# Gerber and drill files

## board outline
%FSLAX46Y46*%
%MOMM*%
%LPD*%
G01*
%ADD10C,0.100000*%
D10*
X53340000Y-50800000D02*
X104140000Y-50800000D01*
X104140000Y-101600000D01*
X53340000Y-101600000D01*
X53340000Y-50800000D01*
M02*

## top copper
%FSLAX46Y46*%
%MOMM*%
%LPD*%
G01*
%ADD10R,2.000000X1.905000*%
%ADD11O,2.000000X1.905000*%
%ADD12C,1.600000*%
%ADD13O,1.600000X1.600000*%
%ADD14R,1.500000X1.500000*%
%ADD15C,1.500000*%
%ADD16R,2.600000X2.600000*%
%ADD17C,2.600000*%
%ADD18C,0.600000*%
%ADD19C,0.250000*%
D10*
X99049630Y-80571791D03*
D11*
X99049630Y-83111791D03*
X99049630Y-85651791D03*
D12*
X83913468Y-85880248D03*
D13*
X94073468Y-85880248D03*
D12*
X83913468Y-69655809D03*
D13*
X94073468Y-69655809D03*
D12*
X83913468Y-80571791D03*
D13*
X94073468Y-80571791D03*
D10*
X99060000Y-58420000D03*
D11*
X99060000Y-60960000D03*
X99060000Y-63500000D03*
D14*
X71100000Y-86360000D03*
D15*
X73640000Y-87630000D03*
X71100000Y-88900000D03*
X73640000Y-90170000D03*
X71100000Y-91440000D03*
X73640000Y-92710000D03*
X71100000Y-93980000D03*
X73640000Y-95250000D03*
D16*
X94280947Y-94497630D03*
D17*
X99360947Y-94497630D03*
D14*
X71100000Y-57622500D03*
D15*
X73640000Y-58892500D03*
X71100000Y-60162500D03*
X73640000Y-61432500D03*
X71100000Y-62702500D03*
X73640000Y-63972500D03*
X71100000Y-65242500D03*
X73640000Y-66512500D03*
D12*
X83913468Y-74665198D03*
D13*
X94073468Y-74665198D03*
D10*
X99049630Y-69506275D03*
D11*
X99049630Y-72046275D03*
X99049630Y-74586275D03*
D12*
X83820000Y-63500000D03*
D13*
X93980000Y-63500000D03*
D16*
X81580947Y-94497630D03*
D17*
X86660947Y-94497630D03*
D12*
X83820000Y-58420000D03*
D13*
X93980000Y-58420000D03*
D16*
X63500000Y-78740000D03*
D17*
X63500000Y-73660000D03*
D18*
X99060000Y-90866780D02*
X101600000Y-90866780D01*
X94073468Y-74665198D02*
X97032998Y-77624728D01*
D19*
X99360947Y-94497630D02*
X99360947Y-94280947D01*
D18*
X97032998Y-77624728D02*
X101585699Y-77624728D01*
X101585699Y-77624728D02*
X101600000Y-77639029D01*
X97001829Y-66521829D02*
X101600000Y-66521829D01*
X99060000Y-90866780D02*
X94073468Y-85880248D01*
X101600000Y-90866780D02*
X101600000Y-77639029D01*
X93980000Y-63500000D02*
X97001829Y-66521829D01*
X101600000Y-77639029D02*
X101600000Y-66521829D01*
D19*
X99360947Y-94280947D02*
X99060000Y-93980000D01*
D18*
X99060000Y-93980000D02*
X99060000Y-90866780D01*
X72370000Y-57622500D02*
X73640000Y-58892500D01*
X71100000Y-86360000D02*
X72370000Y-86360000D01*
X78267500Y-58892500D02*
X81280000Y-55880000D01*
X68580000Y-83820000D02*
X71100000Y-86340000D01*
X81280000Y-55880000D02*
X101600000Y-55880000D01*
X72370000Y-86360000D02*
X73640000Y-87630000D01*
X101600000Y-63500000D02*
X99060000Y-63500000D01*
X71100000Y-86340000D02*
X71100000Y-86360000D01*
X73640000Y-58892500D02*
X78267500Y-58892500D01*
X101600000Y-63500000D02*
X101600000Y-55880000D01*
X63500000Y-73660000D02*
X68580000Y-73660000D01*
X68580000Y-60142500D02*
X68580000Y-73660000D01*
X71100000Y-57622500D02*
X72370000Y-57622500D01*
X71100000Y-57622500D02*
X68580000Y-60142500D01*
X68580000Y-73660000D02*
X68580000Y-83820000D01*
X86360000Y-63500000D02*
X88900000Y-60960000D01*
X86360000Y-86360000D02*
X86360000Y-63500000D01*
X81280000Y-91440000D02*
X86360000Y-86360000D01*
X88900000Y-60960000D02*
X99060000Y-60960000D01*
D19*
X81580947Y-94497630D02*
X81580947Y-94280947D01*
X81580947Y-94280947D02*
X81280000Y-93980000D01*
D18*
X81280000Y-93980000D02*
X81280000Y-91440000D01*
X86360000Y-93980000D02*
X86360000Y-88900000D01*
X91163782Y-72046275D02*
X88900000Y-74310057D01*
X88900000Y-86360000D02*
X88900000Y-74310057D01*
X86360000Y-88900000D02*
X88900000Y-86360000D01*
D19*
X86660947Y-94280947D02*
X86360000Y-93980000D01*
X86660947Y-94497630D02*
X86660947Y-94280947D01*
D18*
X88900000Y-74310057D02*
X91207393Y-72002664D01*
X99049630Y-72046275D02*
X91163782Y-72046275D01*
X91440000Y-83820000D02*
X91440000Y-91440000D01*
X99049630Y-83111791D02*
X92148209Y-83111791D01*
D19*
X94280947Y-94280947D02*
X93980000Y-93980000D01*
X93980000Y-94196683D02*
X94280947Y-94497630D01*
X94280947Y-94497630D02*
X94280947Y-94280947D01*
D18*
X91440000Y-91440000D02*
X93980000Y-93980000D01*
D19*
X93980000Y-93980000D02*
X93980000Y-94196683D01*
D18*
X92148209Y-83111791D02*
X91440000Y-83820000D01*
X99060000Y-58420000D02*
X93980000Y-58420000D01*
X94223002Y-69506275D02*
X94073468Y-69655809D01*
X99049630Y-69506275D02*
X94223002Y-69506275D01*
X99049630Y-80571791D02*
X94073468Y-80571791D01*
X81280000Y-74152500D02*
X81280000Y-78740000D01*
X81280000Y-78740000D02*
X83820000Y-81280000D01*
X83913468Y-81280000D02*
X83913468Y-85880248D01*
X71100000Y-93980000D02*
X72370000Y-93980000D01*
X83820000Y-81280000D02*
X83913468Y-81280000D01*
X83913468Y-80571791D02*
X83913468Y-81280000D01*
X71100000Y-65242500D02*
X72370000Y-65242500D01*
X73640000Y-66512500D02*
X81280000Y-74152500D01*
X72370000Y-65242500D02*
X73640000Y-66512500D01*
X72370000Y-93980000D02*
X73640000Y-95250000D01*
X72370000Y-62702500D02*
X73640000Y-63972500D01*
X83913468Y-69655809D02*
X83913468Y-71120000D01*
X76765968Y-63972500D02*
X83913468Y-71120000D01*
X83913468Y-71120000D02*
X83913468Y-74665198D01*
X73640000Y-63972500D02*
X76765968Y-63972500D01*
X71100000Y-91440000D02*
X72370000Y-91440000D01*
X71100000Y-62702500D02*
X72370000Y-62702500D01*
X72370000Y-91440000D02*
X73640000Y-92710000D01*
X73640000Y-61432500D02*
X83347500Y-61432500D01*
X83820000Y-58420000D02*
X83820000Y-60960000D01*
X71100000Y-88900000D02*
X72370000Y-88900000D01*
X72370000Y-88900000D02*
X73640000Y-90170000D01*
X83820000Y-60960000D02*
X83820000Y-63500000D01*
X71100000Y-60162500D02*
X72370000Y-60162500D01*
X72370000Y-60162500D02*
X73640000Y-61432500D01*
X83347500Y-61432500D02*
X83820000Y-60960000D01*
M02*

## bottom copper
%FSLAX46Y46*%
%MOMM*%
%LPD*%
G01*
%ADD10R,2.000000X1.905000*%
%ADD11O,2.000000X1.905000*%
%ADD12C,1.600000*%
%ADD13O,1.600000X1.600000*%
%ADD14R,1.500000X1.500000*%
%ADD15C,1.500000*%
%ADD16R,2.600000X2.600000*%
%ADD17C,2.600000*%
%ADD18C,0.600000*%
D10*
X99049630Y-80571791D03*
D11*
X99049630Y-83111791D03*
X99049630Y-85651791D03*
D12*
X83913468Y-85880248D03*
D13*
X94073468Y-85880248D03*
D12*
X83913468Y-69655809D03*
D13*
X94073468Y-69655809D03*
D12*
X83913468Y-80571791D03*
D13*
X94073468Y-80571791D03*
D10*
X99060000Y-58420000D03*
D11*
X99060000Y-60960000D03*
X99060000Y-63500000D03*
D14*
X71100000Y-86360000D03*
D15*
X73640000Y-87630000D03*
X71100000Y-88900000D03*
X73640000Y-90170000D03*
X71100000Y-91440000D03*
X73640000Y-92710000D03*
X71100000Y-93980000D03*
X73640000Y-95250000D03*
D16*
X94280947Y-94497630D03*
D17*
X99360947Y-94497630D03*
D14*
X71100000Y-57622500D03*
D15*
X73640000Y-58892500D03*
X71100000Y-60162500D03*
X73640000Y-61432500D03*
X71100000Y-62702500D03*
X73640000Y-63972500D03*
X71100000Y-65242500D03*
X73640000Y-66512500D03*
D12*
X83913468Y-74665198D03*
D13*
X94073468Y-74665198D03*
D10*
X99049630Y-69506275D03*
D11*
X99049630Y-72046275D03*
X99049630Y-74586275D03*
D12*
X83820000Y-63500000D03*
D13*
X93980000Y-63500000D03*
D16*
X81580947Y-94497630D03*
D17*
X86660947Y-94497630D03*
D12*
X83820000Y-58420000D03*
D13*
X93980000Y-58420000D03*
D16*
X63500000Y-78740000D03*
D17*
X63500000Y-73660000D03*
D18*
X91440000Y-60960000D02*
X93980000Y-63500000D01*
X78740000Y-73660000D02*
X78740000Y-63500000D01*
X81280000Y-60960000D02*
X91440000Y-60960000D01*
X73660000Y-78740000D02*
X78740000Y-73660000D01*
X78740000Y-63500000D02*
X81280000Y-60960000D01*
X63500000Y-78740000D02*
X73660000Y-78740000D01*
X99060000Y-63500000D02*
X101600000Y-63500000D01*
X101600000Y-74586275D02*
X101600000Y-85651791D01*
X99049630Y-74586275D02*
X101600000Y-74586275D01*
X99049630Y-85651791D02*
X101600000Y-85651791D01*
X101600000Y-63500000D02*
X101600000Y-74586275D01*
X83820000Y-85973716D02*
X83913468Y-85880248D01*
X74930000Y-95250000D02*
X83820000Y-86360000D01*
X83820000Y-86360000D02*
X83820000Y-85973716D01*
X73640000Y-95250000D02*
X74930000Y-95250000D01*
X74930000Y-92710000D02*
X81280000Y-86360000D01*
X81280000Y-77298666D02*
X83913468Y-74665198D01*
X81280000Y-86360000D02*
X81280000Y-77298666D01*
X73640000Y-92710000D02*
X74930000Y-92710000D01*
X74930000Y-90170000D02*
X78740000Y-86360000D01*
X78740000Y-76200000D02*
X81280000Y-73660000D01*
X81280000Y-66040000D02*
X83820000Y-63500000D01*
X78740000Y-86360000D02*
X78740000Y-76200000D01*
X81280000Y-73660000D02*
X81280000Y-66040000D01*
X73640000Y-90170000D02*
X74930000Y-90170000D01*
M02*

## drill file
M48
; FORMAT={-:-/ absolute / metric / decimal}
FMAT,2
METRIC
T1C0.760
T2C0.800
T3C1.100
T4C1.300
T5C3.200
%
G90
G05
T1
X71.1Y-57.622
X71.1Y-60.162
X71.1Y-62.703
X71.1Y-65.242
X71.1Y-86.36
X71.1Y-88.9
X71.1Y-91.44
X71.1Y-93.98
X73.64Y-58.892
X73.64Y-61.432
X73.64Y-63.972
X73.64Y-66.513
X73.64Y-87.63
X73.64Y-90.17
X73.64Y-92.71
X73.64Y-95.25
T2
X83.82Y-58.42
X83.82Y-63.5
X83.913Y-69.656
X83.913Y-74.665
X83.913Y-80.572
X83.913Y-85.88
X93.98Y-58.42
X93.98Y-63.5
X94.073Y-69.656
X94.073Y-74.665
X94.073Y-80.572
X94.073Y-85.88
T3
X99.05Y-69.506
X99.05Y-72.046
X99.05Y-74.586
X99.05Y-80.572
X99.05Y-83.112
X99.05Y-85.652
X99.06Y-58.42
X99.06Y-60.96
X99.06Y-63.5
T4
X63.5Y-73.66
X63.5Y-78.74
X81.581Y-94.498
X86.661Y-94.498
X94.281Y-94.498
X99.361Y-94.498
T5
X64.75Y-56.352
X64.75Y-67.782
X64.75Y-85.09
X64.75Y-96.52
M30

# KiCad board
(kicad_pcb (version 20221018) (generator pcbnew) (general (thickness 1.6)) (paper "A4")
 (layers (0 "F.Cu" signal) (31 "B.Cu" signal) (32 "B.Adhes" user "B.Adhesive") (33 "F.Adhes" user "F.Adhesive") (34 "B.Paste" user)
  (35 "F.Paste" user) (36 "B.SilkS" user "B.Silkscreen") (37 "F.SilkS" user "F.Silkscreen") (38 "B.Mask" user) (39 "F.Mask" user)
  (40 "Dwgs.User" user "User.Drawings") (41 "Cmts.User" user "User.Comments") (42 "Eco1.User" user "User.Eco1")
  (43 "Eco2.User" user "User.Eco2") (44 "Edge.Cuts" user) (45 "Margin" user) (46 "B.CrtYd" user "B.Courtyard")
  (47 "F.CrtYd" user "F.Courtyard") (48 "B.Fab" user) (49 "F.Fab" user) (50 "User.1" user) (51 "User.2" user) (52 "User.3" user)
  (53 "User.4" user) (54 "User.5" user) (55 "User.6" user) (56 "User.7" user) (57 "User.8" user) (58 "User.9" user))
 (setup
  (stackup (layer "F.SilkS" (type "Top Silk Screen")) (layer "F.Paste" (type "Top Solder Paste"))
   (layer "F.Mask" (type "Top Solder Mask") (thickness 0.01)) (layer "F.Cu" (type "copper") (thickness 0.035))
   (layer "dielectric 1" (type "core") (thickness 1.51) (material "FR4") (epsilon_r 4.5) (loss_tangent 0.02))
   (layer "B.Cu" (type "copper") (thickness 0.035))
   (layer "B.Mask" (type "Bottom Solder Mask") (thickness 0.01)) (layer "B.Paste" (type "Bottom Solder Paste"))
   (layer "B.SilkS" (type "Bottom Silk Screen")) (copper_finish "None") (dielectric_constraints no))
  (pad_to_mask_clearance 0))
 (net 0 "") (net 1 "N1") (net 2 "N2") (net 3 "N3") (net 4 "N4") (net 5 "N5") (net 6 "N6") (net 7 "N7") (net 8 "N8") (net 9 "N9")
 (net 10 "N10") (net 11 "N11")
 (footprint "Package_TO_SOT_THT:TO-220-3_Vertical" (layer "F.Cu") (at 99.04963 80.571791 -90)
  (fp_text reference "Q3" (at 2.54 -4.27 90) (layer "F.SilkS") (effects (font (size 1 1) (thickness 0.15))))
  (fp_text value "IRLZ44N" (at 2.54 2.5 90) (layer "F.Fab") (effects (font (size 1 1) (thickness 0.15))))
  (pad "1" thru_hole rect (at 0 0 270) (size 1.905 2) (drill 1.1) (layers "*.Cu" "*.Mask") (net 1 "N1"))
  (pad "2" thru_hole oval (at 2.54 0 270) (size 1.905 2) (drill 1.1) (layers "*.Cu" "*.Mask") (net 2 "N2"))
  (pad "3" thru_hole oval (at 5.08 0 270) (size 1.905 2) (drill 1.1) (layers "*.Cu" "*.Mask") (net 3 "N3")))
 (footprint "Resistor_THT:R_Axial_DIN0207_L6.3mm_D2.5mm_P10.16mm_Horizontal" (layer "F.Cu") (at 83.913468 85.880248)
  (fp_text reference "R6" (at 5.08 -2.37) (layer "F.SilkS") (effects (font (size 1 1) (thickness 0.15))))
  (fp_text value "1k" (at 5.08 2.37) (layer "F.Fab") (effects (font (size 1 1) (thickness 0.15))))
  (pad "1" thru_hole circle (at 0 0) (size 1.6 1.6) (drill 0.8) (layers "*.Cu" "*.Mask") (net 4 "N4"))
  (pad "2" thru_hole oval (at 10.16 0) (size 1.6 1.6) (drill 0.8) (layers "*.Cu" "*.Mask") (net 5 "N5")))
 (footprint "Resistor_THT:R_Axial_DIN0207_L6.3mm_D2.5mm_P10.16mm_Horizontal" (layer "F.Cu") (at 83.913468 69.655809)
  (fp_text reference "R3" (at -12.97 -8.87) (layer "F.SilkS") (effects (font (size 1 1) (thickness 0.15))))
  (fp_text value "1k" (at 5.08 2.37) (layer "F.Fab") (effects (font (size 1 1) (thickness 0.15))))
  (pad "1" thru_hole circle (at 0 0) (size 1.6 1.6) (drill 0.8) (layers "*.Cu" "*.Mask") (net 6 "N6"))
  (pad "2" thru_hole oval (at 10.16 0) (size 1.6 1.6) (drill 0.8) (layers "*.Cu" "*.Mask") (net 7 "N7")))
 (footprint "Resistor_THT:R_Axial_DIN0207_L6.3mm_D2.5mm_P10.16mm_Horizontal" (layer "F.Cu") (at 83.913468 80.571791)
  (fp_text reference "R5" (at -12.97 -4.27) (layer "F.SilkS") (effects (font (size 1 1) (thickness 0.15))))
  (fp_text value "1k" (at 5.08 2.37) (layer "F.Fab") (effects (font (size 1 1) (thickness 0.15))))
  (pad "1" thru_hole circle (at 0 0) (size 1.6 1.6) (drill 0.8) (layers "*.Cu" "*.Mask") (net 4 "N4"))
  (pad "2" thru_hole oval (at 10.16 0) (size 1.6 1.6) (drill 0.8) (layers "*.Cu" "*.Mask") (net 1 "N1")))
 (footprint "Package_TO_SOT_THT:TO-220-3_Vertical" (layer "F.Cu") (at 99.06 58.42 -90)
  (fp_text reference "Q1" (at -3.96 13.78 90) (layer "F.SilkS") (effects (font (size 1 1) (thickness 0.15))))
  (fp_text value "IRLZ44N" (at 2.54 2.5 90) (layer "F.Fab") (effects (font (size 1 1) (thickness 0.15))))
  (pad "1" thru_hole rect (at 0 0 270) (size 1.905 2) (drill 1.1) (layers "*.Cu" "*.Mask") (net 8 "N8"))
  (pad "2" thru_hole oval (at 2.54 0 270) (size 1.905 2) (drill 1.1) (layers "*.Cu" "*.Mask") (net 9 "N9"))
  (pad "3" thru_hole oval (at 5.08 0 270) (size 1.905 2) (drill 1.1) (layers "*.Cu" "*.Mask") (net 3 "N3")))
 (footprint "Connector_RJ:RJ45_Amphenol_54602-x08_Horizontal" (layer "F.Cu") (at 71.1 86.36 -90)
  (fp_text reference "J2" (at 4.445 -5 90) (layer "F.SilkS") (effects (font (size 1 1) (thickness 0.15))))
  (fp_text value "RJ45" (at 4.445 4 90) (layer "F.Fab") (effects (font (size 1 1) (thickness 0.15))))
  (pad "" np_thru_hole circle (at -1.27 6.35 270) (size 3.2 3.2) (drill 3.2) (layers "*.Cu" "*.Mask"))
  (pad "" np_thru_hole circle (at 10.16 6.35 270) (size 3.2 3.2) (drill 3.2) (layers "*.Cu" "*.Mask"))
  (pad "1" thru_hole rect (at 0 0 270) (size 1.5 1.5) (drill 0.76) (layers "*.Cu" "*.Mask") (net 3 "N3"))
  (pad "2" thru_hole circle (at 1.27 -2.54 270) (size 1.5 1.5) (drill 0.76) (layers "*.Cu" "*.Mask") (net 3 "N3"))
  (pad "3" thru_hole circle (at 2.54 0 270) (size 1.5 1.5) (drill 0.76) (layers "*.Cu" "*.Mask") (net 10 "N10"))
  (pad "4" thru_hole circle (at 3.81 -2.54 270) (size 1.5 1.5) (drill 0.76) (layers "*.Cu" "*.Mask") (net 10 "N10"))
  (pad "5" thru_hole circle (at 5.08 0 270) (size 1.5 1.5) (drill 0.76) (layers "*.Cu" "*.Mask") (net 6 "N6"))
  (pad "6" thru_hole circle (at 6.35 -2.54 270) (size 1.5 1.5) (drill 0.76) (layers "*.Cu" "*.Mask") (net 6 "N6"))
  (pad "7" thru_hole circle (at 7.62 0 270) (size 1.5 1.5) (drill 0.76) (layers "*.Cu" "*.Mask") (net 4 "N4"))
  (pad "8" thru_hole circle (at 8.89 -2.54 270) (size 1.5 1.5) (drill 0.76) (layers "*.Cu" "*.Mask") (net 4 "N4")))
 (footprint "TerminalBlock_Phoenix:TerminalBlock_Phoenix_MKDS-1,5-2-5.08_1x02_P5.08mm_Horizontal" (layer "F.Cu") (at 94.280947 94.49763)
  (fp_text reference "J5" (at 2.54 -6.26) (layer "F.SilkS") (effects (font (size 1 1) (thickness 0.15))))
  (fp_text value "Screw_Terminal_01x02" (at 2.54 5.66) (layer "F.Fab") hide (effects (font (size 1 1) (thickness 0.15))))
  (pad "1" thru_hole rect (at 0 0) (size 2.6 2.6) (drill 1.3) (layers "*.Cu" "*.Mask") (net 2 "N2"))
  (pad "2" thru_hole circle (at 5.08 0) (size 2.6 2.6) (drill 1.3) (layers "*.Cu" "*.Mask") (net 5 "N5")))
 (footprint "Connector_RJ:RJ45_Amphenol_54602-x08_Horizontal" (layer "F.Cu") (at 71.1 57.6225 -90)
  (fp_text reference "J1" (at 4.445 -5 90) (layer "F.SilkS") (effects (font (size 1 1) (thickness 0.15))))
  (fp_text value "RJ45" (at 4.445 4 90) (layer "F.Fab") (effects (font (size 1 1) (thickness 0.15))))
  (pad "" np_thru_hole circle (at -1.27 6.35 270) (size 3.2 3.2) (drill 3.2) (layers "*.Cu" "*.Mask"))
  (pad "" np_thru_hole circle (at 10.16 6.35 270) (size 3.2 3.2) (drill 3.2) (layers "*.Cu" "*.Mask"))
  (pad "1" thru_hole rect (at 0 0 270) (size 1.5 1.5) (drill 0.76) (layers "*.Cu" "*.Mask") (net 3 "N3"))
  (pad "2" thru_hole circle (at 1.27 -2.54 270) (size 1.5 1.5) (drill 0.76) (layers "*.Cu" "*.Mask") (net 3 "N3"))
  (pad "3" thru_hole circle (at 2.54 0 270) (size 1.5 1.5) (drill 0.76) (layers "*.Cu" "*.Mask") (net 10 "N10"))
  (pad "4" thru_hole circle (at 3.81 -2.54 270) (size 1.5 1.5) (drill 0.76) (layers "*.Cu" "*.Mask") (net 10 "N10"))
  (pad "5" thru_hole circle (at 5.08 0 270) (size 1.5 1.5) (drill 0.76) (layers "*.Cu" "*.Mask") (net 6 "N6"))
  (pad "6" thru_hole circle (at 6.35 -2.54 270) (size 1.5 1.5) (drill 0.76) (layers "*.Cu" "*.Mask") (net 6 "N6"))
  (pad "7" thru_hole circle (at 7.62 0 270) (size 1.5 1.5) (drill 0.76) (layers "*.Cu" "*.Mask") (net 4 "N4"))
  (pad "8" thru_hole circle (at 8.89 -2.54 270) (size 1.5 1.5) (drill 0.76) (layers "*.Cu" "*.Mask") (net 4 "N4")))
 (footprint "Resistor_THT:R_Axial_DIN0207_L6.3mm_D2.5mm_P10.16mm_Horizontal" (layer "F.Cu") (at 83.913468 74.665198)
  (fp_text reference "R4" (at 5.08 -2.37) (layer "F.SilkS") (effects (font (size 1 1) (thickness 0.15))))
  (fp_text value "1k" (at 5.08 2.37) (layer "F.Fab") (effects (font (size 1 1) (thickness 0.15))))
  (pad "1" thru_hole circle (at 0 0) (size 1.6 1.6) (drill 0.8) (layers "*.Cu" "*.Mask") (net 6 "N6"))
  (pad "2" thru_hole oval (at 10.16 0) (size 1.6 1.6) (drill 0.8) (layers "*.Cu" "*.Mask") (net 5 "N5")))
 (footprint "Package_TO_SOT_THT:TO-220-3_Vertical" (layer "F.Cu") (at 99.04963 69.506275 -90)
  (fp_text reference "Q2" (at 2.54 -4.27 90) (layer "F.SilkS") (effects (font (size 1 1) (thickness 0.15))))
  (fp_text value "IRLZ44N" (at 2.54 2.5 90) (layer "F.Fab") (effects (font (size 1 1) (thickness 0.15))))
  (pad "1" thru_hole rect (at 0 0 270) (size 1.905 2) (drill 1.1) (layers "*.Cu" "*.Mask") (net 7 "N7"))
  (pad "2" thru_hole oval (at 2.54 0 270) (size 1.905 2) (drill 1.1) (layers "*.Cu" "*.Mask") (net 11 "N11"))
  (pad "3" thru_hole oval (at 5.08 0 270) (size 1.905 2) (drill 1.1) (layers "*.Cu" "*.Mask") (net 3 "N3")))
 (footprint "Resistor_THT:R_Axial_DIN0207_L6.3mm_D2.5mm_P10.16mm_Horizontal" (layer "F.Cu") (at 83.82 63.5)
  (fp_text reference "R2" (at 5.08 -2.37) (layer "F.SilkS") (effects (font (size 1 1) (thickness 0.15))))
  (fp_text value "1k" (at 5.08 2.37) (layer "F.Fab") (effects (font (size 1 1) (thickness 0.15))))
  (pad "1" thru_hole circle (at 0 0) (size 1.6 1.6) (drill 0.8) (layers "*.Cu" "*.Mask") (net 10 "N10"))
  (pad "2" thru_hole oval (at 10.16 0) (size 1.6 1.6) (drill 0.8) (layers "*.Cu" "*.Mask") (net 5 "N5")))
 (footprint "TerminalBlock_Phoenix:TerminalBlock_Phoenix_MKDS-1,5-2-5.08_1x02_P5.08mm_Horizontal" (layer "F.Cu") (at 81.580947 94.49763)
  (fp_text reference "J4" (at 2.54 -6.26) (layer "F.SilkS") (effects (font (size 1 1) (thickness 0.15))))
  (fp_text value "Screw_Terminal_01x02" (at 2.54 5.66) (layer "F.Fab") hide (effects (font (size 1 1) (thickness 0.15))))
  (pad "1" thru_hole rect (at 0 0) (size 2.6 2.6) (drill 1.3) (layers "*.Cu" "*.Mask") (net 9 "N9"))
  (pad "2" thru_hole circle (at 5.08 0) (size 2.6 2.6) (drill 1.3) (layers "*.Cu" "*.Mask") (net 11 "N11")))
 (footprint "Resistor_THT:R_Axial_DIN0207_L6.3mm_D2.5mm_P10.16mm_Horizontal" (layer "F.Cu") (at 83.82 58.42)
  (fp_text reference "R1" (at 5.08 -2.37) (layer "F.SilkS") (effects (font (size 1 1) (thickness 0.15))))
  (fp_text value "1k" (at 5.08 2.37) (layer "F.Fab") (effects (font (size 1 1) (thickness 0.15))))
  (pad "1" thru_hole circle (at 0 0) (size 1.6 1.6) (drill 0.8) (layers "*.Cu" "*.Mask") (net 10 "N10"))
  (pad "2" thru_hole oval (at 10.16 0) (size 1.6 1.6) (drill 0.8) (layers "*.Cu" "*.Mask") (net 8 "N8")))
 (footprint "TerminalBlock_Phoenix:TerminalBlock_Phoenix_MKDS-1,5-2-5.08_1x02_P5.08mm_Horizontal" (layer "F.Cu") (at 63.5 78.74 90)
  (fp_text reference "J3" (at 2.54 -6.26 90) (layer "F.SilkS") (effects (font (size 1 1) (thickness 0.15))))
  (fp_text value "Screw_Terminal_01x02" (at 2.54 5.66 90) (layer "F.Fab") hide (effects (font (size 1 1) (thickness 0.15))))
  (pad "1" thru_hole rect (at 0 0 90) (size 2.6 2.6) (drill 1.3) (layers "*.Cu" "*.Mask") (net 5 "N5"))
  (pad "2" thru_hole circle (at 5.08 0 90) (size 2.6 2.6) (drill 1.3) (layers "*.Cu" "*.Mask") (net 3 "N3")))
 (gr_rect (start 53.34 50.8) (end 104.14 101.6) (stroke (width 0.1) (type default)) (fill none) (layer "Edge.Cuts"))
 (segment (start 99.06 90.86678) (end 101.6 90.86678) (width 0.6) (layer "F.Cu") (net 5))
 (segment (start 94.073468 74.665198) (end 97.032998 77.624728) (width 0.6) (layer "F.Cu") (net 5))
 (segment (start 99.360947 94.49763) (end 99.360947 94.280947) (width 0.25) (layer "F.Cu") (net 5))
 (segment (start 97.032998 77.624728) (end 101.585699 77.624728) (width 0.6) (layer "F.Cu") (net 5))
 (segment (start 101.585699 77.624728) (end 101.6 77.639029) (width 0.6) (layer "F.Cu") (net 5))
 (segment (start 97.001829 66.521829) (end 101.6 66.521829) (width 0.6) (layer "F.Cu") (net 5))
 (segment (start 99.06 90.86678) (end 94.073468 85.880248) (width 0.6) (layer "F.Cu") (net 5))
 (segment (start 101.6 90.86678) (end 101.6 77.639029) (width 0.6) (layer "F.Cu") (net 5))
 (segment (start 93.98 63.5) (end 97.001829 66.521829) (width 0.6) (layer "F.Cu") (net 5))
 (segment (start 101.6 77.639029) (end 101.6 66.521829) (width 0.6) (layer "F.Cu") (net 5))
 (segment (start 99.360947 94.280947) (end 99.06 93.98) (width 0.25) (layer "F.Cu") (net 5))
 (segment (start 99.06 93.98) (end 99.06 90.86678) (width 0.6) (layer "F.Cu") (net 5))
 (segment (start 91.44 60.96) (end 93.98 63.5) (width 0.6) (layer "B.Cu") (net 5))
 (segment (start 78.74 73.66) (end 78.74 63.5) (width 0.6) (layer "B.Cu") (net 5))
 (segment (start 81.28 60.96) (end 91.44 60.96) (width 0.6) (layer "B.Cu") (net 5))
 (segment (start 73.66 78.74) (end 78.74 73.66) (width 0.6) (layer "B.Cu") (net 5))
 (segment (start 78.74 63.5) (end 81.28 60.96) (width 0.6) (layer "B.Cu") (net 5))
 (segment (start 63.5 78.74) (end 73.66 78.74) (width 0.6) (layer "B.Cu") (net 5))
 (segment (start 72.37 57.6225) (end 73.64 58.8925) (width 0.6) (layer "F.Cu") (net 3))
 (segment (start 71.1 86.36) (end 72.37 86.36) (width 0.6) (layer "F.Cu") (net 3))
 (segment (start 78.2675 58.8925) (end 81.28 55.88) (width 0.6) (layer "F.Cu") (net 3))
 (segment (start 68.58 83.82) (end 71.1 86.34) (width 0.6) (layer "F.Cu") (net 3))
 (segment (start 81.28 55.88) (end 101.6 55.88) (width 0.6) (layer "F.Cu") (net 3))
 (segment (start 72.37 86.36) (end 73.64 87.63) (width 0.6) (layer "F.Cu") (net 3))
 (segment (start 101.6 63.5) (end 99.06 63.5) (width 0.6) (layer "F.Cu") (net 3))
 (segment (start 71.1 86.34) (end 71.1 86.36) (width 0.6) (layer "F.Cu") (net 3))
 (segment (start 73.64 58.8925) (end 78.2675 58.8925) (width 0.6) (layer "F.Cu") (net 3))
 (segment (start 101.6 63.5) (end 101.6 55.88) (width 0.6) (layer "F.Cu") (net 3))
 (segment (start 63.5 73.66) (end 68.58 73.66) (width 0.6) (layer "F.Cu") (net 3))
 (segment (start 68.58 60.1425) (end 68.58 73.66) (width 0.6) (layer "F.Cu") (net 3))
 (segment (start 71.1 57.6225) (end 72.37 57.6225) (width 0.6) (layer "F.Cu") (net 3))
 (segment (start 71.1 57.6225) (end 68.58 60.1425) (width 0.6) (layer "F.Cu") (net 3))
 (segment (start 68.58 73.66) (end 68.58 83.82) (width 0.6) (layer "F.Cu") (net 3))
 (segment (start 99.06 63.5) (end 101.6 63.5) (width 0.6) (layer "B.Cu") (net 3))
 (segment (start 101.6 74.586275) (end 101.6 85.651791) (width 0.6) (layer "B.Cu") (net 3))
 (segment (start 99.04963 74.586275) (end 101.6 74.586275) (width 0.6) (layer "B.Cu") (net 3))
 (segment (start 99.04963 85.651791) (end 101.6 85.651791) (width 0.6) (layer "B.Cu") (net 3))
 (segment (start 101.6 63.5) (end 101.6 74.586275) (width 0.6) (layer "B.Cu") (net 3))
 (segment (start 86.36 63.5) (end 88.9 60.96) (width 0.6) (layer "F.Cu") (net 9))
 (segment (start 86.36 86.36) (end 86.36 63.5) (width 0.6) (layer "F.Cu") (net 9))
 (segment (start 81.28 91.44) (end 86.36 86.36) (width 0.6) (layer "F.Cu") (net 9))
 (segment (start 88.9 60.96) (end 99.06 60.96) (width 0.6) (layer "F.Cu") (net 9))
 (segment (start 81.580947 94.49763) (end 81.580947 94.280947) (width 0.25) (layer "F.Cu") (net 9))
 (segment (start 81.580947 94.280947) (end 81.28 93.98) (width 0.25) (layer "F.Cu") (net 9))
 (segment (start 81.28 93.98) (end 81.28 91.44) (width 0.6) (layer "F.Cu") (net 9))
 (segment (start 86.36 93.98) (end 86.36 88.9) (width 0.6) (layer "F.Cu") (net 11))
 (segment (start 91.163782 72.046275) (end 88.9 74.310057) (width 0.6) (layer "F.Cu") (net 11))
 (segment (start 88.9 86.36) (end 88.9 74.310057) (width 0.6) (layer "F.Cu") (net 11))
 (segment (start 86.36 88.9) (end 88.9 86.36) (width 0.6) (layer "F.Cu") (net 11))
 (segment (start 86.660947 94.280947) (end 86.36 93.98) (width 0.25) (layer "F.Cu") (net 11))
 (segment (start 86.660947 94.49763) (end 86.660947 94.280947) (width 0.25) (layer "F.Cu") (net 11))
 (segment (start 88.9 74.310057) (end 91.207393 72.002664) (width 0.6) (layer "F.Cu") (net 11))
 (segment (start 99.04963 72.046275) (end 91.163782 72.046275) (width 0.6) (layer "F.Cu") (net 11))
 (segment (start 91.44 83.82) (end 91.44 91.44) (width 0.6) (layer "F.Cu") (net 2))
 (segment (start 99.04963 83.111791) (end 92.148209 83.111791) (width 0.6) (layer "F.Cu") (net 2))
 (segment (start 94.280947 94.280947) (end 93.98 93.98) (width 0.25) (layer "F.Cu") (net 2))
 (segment (start 93.98 94.196683) (end 94.280947 94.49763) (width 0.25) (layer "F.Cu") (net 2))
 (segment (start 94.280947 94.49763) (end 94.280947 94.280947) (width 0.25) (layer "F.Cu") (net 2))
 (segment (start 91.44 91.44) (end 93.98 93.98) (width 0.6) (layer "F.Cu") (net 2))
 (segment (start 93.98 93.98) (end 93.98 94.196683) (width 0.25) (layer "F.Cu") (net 2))
 (segment (start 92.148209 83.111791) (end 91.44 83.82) (width 0.6) (layer "F.Cu") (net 2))
 (segment (start 99.06 58.42) (end 93.98 58.42) (width 0.6) (layer "F.Cu") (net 8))
 (segment (start 94.223002 69.506275) (end 94.073468 69.655809) (width 0.6) (layer "F.Cu") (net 7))
 (segment (start 99.04963 69.506275) (end 94.223002 69.506275) (width 0.6) (layer "F.Cu") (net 7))
 (segment (start 99.04963 80.571791) (end 94.073468 80.571791) (width 0.6) (layer "F.Cu") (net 1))
 (segment (start 81.28 74.1525) (end 81.28 78.74) (width 0.6) (layer "F.Cu") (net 4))
 (segment (start 81.28 78.74) (end 83.82 81.28) (width 0.6) (layer "F.Cu") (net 4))
 (segment (start 83.913468 81.28) (end 83.913468 85.880248) (width 0.6) (layer "F.Cu") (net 4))
 (segment (start 71.1 93.98) (end 72.37 93.98) (width 0.6) (layer "F.Cu") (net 4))
 (segment (start 83.82 81.28) (end 83.913468 81.28) (width 0.6) (layer "F.Cu") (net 4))
 (segment (start 83.913468 80.571791) (end 83.913468 81.28) (width 0.6) (layer "F.Cu") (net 4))
 (segment (start 71.1 65.2425) (end 72.37 65.2425) (width 0.6) (layer "F.Cu") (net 4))
 (segment (start 73.64 66.5125) (end 81.28 74.1525) (width 0.6) (layer "F.Cu") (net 4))
 (segment (start 72.37 65.2425) (end 73.64 66.5125) (width 0.6) (layer "F.Cu") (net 4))
 (segment (start 72.37 93.98) (end 73.64 95.25) (width 0.6) (layer "F.Cu") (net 4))
 (segment (start 83.82 85.973716) (end 83.913468 85.880248) (width 0.6) (layer "B.Cu") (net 4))
 (segment (start 74.93 95.25) (end 83.82 86.36) (width 0.6) (layer "B.Cu") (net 4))
 (segment (start 83.82 86.36) (end 83.82 85.973716) (width 0.6) (layer "B.Cu") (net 4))
 (segment (start 73.64 95.25) (end 74.93 95.25) (width 0.6) (layer "B.Cu") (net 4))
 (segment (start 72.37 62.7025) (end 73.64 63.9725) (width 0.6) (layer "F.Cu") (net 6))
 (segment (start 83.913468 69.655809) (end 83.913468 71.12) (width 0.6) (layer "F.Cu") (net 6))
 (segment (start 76.765968 63.9725) (end 83.913468 71.12) (width 0.6) (layer "F.Cu") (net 6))
 (segment (start 83.913468 71.12) (end 83.913468 74.665198) (width 0.6) (layer "F.Cu") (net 6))
 (segment (start 73.64 63.9725) (end 76.765968 63.9725) (width 0.6) (layer "F.Cu") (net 6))
 (segment (start 71.1 91.44) (end 72.37 91.44) (width 0.6) (layer "F.Cu") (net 6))
 (segment (start 71.1 62.7025) (end 72.37 62.7025) (width 0.6) (layer "F.Cu") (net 6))
 (segment (start 72.37 91.44) (end 73.64 92.71) (width 0.6) (layer "F.Cu") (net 6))
 (segment (start 74.93 92.71) (end 81.28 86.36) (width 0.6) (layer "B.Cu") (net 6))
 (segment (start 81.28 77.298666) (end 83.913468 74.665198) (width 0.6) (layer "B.Cu") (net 6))
 (segment (start 81.28 86.36) (end 81.28 77.298666) (width 0.6) (layer "B.Cu") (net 6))
 (segment (start 73.64 92.71) (end 74.93 92.71) (width 0.6) (layer "B.Cu") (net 6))
 (segment (start 73.64 61.4325) (end 83.3475 61.4325) (width 0.6) (layer "F.Cu") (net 10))
 (segment (start 83.82 58.42) (end 83.82 60.96) (width 0.6) (layer "F.Cu") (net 10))
 (segment (start 71.1 88.9) (end 72.37 88.9) (width 0.6) (layer "F.Cu") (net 10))
 (segment (start 72.37 88.9) (end 73.64 90.17) (width 0.6) (layer "F.Cu") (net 10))
 (segment (start 83.82 60.96) (end 83.82 63.5) (width 0.6) (layer "F.Cu") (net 10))
 (segment (start 71.1 60.1625) (end 72.37 60.1625) (width 0.6) (layer "F.Cu") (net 10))
 (segment (start 72.37 60.1625) (end 73.64 61.4325) (width 0.6) (layer "F.Cu") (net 10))
 (segment (start 83.3475 61.4325) (end 83.82 60.96) (width 0.6) (layer "F.Cu") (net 10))
 (segment (start 74.93 90.17) (end 78.74 86.36) (width 0.6) (layer "B.Cu") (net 10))
 (segment (start 78.74 76.2) (end 81.28 73.66) (width 0.6) (layer "B.Cu") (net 10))
 (segment (start 81.28 66.04) (end 83.82 63.5) (width 0.6) (layer "B.Cu") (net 10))
 (segment (start 78.74 86.36) (end 78.74 76.2) (width 0.6) (layer "B.Cu") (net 10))
 (segment (start 81.28 73.66) (end 81.28 66.04) (width 0.6) (layer "B.Cu") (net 10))
 (segment (start 73.64 90.17) (end 74.93 90.17) (width 0.6) (layer "B.Cu") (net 10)))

